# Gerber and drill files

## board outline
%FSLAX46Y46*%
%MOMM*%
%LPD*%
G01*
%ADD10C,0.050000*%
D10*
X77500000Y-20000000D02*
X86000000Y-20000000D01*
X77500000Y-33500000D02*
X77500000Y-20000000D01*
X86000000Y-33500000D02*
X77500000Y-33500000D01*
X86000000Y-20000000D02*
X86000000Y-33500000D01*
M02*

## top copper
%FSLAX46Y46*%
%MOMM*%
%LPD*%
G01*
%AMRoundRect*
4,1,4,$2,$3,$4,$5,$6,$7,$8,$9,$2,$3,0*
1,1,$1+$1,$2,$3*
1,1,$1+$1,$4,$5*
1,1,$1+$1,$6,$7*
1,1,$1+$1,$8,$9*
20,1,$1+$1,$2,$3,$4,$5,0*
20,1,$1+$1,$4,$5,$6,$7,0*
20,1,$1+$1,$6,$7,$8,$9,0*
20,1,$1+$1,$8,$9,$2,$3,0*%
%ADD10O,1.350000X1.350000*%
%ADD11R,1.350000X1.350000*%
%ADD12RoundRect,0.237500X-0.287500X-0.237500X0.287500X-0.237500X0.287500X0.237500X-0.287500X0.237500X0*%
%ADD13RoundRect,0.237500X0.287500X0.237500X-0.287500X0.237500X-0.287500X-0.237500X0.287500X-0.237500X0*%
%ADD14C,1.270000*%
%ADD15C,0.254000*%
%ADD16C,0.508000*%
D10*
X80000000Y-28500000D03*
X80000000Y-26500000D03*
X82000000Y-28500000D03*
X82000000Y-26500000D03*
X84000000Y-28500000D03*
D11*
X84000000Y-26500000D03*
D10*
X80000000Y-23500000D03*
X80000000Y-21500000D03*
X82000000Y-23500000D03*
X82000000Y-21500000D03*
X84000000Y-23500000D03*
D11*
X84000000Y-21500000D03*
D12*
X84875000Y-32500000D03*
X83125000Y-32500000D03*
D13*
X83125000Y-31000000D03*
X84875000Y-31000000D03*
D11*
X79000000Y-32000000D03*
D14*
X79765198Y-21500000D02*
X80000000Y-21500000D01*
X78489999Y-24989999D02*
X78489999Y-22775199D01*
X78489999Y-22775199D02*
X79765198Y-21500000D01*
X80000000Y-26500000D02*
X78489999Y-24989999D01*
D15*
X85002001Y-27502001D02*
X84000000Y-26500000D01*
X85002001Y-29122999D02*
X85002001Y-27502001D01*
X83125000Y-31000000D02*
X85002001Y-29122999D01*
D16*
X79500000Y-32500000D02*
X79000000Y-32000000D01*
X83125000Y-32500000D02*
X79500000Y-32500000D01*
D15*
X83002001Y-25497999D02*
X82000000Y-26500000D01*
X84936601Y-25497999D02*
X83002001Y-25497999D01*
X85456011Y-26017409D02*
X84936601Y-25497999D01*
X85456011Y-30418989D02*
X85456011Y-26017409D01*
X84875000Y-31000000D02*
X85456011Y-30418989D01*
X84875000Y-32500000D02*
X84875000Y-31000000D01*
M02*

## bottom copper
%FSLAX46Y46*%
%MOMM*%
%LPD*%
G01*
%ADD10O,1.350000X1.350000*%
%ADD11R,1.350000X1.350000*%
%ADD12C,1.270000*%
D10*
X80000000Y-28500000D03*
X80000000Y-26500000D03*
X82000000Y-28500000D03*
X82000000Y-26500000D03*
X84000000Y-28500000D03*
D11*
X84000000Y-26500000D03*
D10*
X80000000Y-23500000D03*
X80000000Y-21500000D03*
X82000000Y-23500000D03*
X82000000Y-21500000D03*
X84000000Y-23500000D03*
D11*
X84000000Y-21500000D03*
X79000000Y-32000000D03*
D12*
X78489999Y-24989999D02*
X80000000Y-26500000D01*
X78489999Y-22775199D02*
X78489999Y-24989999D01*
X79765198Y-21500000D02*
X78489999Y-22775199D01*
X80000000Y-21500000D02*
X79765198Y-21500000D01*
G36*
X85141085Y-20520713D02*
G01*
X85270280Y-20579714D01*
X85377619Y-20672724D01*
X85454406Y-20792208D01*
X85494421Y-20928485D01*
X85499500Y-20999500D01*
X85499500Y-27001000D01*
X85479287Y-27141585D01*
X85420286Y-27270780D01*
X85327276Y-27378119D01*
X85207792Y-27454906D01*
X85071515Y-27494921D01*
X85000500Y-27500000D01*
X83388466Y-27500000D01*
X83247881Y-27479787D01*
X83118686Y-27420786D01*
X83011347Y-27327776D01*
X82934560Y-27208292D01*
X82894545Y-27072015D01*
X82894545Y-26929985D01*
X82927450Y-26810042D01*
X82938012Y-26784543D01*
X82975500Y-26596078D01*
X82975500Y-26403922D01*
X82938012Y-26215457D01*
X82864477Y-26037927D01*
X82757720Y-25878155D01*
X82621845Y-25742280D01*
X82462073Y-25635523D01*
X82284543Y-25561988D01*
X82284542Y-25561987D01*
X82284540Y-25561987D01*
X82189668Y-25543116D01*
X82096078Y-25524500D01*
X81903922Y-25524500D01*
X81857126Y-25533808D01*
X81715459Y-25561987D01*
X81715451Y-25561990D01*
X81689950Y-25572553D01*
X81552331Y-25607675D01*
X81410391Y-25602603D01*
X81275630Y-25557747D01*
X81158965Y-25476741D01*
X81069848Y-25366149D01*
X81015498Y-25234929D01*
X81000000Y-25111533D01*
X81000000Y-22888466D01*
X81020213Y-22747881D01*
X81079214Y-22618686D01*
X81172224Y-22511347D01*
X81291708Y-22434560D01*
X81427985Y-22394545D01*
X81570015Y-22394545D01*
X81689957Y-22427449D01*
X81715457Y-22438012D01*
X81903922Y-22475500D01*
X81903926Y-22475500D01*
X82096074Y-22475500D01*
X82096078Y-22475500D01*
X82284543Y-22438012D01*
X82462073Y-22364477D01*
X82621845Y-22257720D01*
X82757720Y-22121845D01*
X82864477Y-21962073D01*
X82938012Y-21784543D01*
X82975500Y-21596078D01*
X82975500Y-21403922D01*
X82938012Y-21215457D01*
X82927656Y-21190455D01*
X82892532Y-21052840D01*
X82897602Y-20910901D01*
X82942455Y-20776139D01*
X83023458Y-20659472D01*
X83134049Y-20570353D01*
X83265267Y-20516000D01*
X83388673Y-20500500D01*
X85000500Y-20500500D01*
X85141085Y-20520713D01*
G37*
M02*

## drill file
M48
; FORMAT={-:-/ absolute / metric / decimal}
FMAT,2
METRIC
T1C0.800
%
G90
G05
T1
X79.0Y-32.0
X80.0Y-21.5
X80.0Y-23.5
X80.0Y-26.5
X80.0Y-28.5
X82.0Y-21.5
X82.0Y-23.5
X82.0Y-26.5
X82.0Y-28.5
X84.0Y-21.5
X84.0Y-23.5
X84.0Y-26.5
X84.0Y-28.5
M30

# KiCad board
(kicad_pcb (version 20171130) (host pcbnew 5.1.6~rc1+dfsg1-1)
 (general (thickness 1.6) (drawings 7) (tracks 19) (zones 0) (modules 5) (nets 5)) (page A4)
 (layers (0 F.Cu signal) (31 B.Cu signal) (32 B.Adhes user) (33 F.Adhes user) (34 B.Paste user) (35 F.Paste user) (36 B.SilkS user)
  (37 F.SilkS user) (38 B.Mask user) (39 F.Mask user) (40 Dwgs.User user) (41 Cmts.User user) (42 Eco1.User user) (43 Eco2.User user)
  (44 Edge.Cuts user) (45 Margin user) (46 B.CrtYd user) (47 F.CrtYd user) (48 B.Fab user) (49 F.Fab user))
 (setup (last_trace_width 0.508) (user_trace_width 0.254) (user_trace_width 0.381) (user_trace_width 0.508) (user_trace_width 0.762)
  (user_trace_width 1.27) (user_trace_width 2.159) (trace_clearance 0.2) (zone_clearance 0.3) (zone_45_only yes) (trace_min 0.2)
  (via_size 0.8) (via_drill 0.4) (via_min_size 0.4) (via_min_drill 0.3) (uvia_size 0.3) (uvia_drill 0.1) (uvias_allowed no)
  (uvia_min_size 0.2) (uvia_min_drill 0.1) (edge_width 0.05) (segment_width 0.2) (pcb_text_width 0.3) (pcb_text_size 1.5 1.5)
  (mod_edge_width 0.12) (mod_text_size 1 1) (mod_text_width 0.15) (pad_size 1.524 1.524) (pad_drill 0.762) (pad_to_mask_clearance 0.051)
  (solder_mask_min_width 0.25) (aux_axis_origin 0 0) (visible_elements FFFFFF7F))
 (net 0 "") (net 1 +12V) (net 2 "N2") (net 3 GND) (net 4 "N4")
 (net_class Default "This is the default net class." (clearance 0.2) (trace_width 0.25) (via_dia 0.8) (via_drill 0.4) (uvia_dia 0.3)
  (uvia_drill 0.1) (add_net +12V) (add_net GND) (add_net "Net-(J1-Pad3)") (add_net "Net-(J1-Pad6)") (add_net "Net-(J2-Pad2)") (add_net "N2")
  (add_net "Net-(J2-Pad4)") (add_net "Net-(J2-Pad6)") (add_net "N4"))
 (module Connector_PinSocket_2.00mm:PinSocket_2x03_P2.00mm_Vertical (layer B.Cu) (at 84 26.5 90)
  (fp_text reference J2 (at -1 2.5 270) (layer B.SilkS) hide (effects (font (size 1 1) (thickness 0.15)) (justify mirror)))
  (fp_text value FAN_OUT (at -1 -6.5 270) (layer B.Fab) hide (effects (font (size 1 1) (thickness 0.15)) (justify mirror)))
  (pad 6 thru_hole oval (at -2 -4 90) (size 1.35 1.35) (drill 0.8) (layers *.Cu *.Mask))
  (pad 5 thru_hole oval (at 0 -4 90) (size 1.35 1.35) (drill 0.8) (layers *.Cu *.Mask) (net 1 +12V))
  (pad 4 thru_hole oval (at -2 -2 90) (size 1.35 1.35) (drill 0.8) (layers *.Cu *.Mask))
  (pad 3 thru_hole oval (at 0 -2 90) (size 1.35 1.35) (drill 0.8) (layers *.Cu *.Mask) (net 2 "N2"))
  (pad 2 thru_hole oval (at -2 0 90) (size 1.35 1.35) (drill 0.8) (layers *.Cu *.Mask))
  (pad 1 thru_hole rect (at 0 0 90) (size 1.35 1.35) (drill 0.8) (layers *.Cu *.Mask) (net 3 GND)))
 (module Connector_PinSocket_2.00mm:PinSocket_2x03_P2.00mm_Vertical (layer B.Cu) (at 84 21.5 90)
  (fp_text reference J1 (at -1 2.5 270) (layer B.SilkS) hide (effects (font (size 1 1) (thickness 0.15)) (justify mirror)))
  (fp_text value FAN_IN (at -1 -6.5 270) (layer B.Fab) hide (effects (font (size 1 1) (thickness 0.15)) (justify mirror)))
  (pad 6 thru_hole oval (at -2 -4 90) (size 1.35 1.35) (drill 0.8) (layers *.Cu *.Mask))
  (pad 5 thru_hole oval (at 0 -4 90) (size 1.35 1.35) (drill 0.8) (layers *.Cu *.Mask) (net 1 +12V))
  (pad 4 thru_hole oval (at -2 -2 90) (size 1.35 1.35) (drill 0.8) (layers *.Cu *.Mask) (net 3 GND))
  (pad 3 thru_hole oval (at 0 -2 90) (size 1.35 1.35) (drill 0.8) (layers *.Cu *.Mask))
  (pad 2 thru_hole oval (at -2 0 90) (size 1.35 1.35) (drill 0.8) (layers *.Cu *.Mask) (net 3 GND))
  (pad 1 thru_hole rect (at 0 0 90) (size 1.35 1.35) (drill 0.8) (layers *.Cu *.Mask) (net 3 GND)))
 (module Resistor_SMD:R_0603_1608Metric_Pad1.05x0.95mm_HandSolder (layer F.Cu) (at 84 32.5)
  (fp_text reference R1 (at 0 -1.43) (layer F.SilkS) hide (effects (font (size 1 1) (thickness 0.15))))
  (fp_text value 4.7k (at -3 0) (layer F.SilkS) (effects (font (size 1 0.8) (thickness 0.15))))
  (pad 2 smd roundrect (at 0.875 0) (size 1.05 0.95) (layers F.Cu F.Paste F.Mask) (roundrect_rratio 0.25) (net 2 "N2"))
  (pad 1 smd roundrect (at -0.875 0) (size 1.05 0.95) (layers F.Cu F.Paste F.Mask) (roundrect_rratio 0.25) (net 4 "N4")))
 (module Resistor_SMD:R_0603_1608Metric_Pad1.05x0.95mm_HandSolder (layer F.Cu) (at 84 31 180)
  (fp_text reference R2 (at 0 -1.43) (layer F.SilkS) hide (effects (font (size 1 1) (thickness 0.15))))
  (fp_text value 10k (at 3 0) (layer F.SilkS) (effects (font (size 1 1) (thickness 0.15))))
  (pad 2 smd roundrect (at 0.875 0 180) (size 1.05 0.95) (layers F.Cu F.Paste F.Mask) (roundrect_rratio 0.25) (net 3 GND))
  (pad 1 smd roundrect (at -0.875 0 180) (size 1.05 0.95) (layers F.Cu F.Paste F.Mask) (roundrect_rratio 0.25) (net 2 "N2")))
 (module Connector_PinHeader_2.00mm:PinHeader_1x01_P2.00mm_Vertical (layer F.Cu) (at 79 32)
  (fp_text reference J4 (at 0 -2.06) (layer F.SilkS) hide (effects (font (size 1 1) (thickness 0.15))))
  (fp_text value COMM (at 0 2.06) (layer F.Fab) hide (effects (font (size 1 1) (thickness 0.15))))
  (pad 1 thru_hole rect (at 0 0) (size 1.35 1.35) (drill 0.8) (layers *.Cu *.Mask) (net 4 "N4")))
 (gr_line (start 77.5 20) (end 86 20) (layer Edge.Cuts) (width 0.05))
 (gr_line (start 77.5 33.5) (end 77.5 20) (layer Edge.Cuts) (width 0.05))
 (gr_line (start 86 33.5) (end 77.5 33.5) (layer Edge.Cuts) (width 0.05))
 (gr_line (start 86 20) (end 86 33.5) (layer Edge.Cuts) (width 0.05))
 (segment (start 78.489999 24.989999) (end 80 26.5) (width 1.27) (layer B.Cu) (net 1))
 (segment (start 78.489999 22.775199) (end 78.489999 24.989999) (width 1.27) (layer B.Cu) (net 1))
 (segment (start 79.765198 21.5) (end 78.489999 22.775199) (width 1.27) (layer B.Cu) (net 1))
 (segment (start 80 21.5) (end 79.765198 21.5) (width 1.27) (layer B.Cu) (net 1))
 (segment (start 79.765198 21.5) (end 80 21.5) (width 1.27) (layer F.Cu) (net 1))
 (segment (start 78.489999 24.989999) (end 78.489999 22.775199) (width 1.27) (layer F.Cu) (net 1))
 (segment (start 78.489999 22.775199) (end 79.765198 21.5) (width 1.27) (layer F.Cu) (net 1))
 (segment (start 80 26.5) (end 78.489999 24.989999) (width 1.27) (layer F.Cu) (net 1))
 (segment (start 85.002001 27.502001) (end 84 26.5) (width 0.254) (layer F.Cu) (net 3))
 (segment (start 85.002001 29.122999) (end 85.002001 27.502001) (width 0.254) (layer F.Cu) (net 3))
 (segment (start 83.125 31) (end 85.002001 29.122999) (width 0.254) (layer F.Cu) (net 3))
 (segment (start 79.5 32.5) (end 79 32) (width 0.508) (layer F.Cu) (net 4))
 (segment (start 83.125 32.5) (end 79.5 32.5) (width 0.508) (layer F.Cu) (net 4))
 (segment (start 83.002001 25.497999) (end 82 26.5) (width 0.254) (layer F.Cu) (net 2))
 (segment (start 84.936601 25.497999) (end 83.002001 25.497999) (width 0.254) (layer F.Cu) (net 2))
 (segment (start 85.456011 26.017409) (end 84.936601 25.497999) (width 0.254) (layer F.Cu) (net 2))
 (segment (start 85.456011 30.418989) (end 85.456011 26.017409) (width 0.254) (layer F.Cu) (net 2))
 (segment (start 84.875 31) (end 85.456011 30.418989) (width 0.254) (layer F.Cu) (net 2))
 (segment (start 84.875 32.5) (end 84.875 31) (width 0.254) (layer F.Cu) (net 2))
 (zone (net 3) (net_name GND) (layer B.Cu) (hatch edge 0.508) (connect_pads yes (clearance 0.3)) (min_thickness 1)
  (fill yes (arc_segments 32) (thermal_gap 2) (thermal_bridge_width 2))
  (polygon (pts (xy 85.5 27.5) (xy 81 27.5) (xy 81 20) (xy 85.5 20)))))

